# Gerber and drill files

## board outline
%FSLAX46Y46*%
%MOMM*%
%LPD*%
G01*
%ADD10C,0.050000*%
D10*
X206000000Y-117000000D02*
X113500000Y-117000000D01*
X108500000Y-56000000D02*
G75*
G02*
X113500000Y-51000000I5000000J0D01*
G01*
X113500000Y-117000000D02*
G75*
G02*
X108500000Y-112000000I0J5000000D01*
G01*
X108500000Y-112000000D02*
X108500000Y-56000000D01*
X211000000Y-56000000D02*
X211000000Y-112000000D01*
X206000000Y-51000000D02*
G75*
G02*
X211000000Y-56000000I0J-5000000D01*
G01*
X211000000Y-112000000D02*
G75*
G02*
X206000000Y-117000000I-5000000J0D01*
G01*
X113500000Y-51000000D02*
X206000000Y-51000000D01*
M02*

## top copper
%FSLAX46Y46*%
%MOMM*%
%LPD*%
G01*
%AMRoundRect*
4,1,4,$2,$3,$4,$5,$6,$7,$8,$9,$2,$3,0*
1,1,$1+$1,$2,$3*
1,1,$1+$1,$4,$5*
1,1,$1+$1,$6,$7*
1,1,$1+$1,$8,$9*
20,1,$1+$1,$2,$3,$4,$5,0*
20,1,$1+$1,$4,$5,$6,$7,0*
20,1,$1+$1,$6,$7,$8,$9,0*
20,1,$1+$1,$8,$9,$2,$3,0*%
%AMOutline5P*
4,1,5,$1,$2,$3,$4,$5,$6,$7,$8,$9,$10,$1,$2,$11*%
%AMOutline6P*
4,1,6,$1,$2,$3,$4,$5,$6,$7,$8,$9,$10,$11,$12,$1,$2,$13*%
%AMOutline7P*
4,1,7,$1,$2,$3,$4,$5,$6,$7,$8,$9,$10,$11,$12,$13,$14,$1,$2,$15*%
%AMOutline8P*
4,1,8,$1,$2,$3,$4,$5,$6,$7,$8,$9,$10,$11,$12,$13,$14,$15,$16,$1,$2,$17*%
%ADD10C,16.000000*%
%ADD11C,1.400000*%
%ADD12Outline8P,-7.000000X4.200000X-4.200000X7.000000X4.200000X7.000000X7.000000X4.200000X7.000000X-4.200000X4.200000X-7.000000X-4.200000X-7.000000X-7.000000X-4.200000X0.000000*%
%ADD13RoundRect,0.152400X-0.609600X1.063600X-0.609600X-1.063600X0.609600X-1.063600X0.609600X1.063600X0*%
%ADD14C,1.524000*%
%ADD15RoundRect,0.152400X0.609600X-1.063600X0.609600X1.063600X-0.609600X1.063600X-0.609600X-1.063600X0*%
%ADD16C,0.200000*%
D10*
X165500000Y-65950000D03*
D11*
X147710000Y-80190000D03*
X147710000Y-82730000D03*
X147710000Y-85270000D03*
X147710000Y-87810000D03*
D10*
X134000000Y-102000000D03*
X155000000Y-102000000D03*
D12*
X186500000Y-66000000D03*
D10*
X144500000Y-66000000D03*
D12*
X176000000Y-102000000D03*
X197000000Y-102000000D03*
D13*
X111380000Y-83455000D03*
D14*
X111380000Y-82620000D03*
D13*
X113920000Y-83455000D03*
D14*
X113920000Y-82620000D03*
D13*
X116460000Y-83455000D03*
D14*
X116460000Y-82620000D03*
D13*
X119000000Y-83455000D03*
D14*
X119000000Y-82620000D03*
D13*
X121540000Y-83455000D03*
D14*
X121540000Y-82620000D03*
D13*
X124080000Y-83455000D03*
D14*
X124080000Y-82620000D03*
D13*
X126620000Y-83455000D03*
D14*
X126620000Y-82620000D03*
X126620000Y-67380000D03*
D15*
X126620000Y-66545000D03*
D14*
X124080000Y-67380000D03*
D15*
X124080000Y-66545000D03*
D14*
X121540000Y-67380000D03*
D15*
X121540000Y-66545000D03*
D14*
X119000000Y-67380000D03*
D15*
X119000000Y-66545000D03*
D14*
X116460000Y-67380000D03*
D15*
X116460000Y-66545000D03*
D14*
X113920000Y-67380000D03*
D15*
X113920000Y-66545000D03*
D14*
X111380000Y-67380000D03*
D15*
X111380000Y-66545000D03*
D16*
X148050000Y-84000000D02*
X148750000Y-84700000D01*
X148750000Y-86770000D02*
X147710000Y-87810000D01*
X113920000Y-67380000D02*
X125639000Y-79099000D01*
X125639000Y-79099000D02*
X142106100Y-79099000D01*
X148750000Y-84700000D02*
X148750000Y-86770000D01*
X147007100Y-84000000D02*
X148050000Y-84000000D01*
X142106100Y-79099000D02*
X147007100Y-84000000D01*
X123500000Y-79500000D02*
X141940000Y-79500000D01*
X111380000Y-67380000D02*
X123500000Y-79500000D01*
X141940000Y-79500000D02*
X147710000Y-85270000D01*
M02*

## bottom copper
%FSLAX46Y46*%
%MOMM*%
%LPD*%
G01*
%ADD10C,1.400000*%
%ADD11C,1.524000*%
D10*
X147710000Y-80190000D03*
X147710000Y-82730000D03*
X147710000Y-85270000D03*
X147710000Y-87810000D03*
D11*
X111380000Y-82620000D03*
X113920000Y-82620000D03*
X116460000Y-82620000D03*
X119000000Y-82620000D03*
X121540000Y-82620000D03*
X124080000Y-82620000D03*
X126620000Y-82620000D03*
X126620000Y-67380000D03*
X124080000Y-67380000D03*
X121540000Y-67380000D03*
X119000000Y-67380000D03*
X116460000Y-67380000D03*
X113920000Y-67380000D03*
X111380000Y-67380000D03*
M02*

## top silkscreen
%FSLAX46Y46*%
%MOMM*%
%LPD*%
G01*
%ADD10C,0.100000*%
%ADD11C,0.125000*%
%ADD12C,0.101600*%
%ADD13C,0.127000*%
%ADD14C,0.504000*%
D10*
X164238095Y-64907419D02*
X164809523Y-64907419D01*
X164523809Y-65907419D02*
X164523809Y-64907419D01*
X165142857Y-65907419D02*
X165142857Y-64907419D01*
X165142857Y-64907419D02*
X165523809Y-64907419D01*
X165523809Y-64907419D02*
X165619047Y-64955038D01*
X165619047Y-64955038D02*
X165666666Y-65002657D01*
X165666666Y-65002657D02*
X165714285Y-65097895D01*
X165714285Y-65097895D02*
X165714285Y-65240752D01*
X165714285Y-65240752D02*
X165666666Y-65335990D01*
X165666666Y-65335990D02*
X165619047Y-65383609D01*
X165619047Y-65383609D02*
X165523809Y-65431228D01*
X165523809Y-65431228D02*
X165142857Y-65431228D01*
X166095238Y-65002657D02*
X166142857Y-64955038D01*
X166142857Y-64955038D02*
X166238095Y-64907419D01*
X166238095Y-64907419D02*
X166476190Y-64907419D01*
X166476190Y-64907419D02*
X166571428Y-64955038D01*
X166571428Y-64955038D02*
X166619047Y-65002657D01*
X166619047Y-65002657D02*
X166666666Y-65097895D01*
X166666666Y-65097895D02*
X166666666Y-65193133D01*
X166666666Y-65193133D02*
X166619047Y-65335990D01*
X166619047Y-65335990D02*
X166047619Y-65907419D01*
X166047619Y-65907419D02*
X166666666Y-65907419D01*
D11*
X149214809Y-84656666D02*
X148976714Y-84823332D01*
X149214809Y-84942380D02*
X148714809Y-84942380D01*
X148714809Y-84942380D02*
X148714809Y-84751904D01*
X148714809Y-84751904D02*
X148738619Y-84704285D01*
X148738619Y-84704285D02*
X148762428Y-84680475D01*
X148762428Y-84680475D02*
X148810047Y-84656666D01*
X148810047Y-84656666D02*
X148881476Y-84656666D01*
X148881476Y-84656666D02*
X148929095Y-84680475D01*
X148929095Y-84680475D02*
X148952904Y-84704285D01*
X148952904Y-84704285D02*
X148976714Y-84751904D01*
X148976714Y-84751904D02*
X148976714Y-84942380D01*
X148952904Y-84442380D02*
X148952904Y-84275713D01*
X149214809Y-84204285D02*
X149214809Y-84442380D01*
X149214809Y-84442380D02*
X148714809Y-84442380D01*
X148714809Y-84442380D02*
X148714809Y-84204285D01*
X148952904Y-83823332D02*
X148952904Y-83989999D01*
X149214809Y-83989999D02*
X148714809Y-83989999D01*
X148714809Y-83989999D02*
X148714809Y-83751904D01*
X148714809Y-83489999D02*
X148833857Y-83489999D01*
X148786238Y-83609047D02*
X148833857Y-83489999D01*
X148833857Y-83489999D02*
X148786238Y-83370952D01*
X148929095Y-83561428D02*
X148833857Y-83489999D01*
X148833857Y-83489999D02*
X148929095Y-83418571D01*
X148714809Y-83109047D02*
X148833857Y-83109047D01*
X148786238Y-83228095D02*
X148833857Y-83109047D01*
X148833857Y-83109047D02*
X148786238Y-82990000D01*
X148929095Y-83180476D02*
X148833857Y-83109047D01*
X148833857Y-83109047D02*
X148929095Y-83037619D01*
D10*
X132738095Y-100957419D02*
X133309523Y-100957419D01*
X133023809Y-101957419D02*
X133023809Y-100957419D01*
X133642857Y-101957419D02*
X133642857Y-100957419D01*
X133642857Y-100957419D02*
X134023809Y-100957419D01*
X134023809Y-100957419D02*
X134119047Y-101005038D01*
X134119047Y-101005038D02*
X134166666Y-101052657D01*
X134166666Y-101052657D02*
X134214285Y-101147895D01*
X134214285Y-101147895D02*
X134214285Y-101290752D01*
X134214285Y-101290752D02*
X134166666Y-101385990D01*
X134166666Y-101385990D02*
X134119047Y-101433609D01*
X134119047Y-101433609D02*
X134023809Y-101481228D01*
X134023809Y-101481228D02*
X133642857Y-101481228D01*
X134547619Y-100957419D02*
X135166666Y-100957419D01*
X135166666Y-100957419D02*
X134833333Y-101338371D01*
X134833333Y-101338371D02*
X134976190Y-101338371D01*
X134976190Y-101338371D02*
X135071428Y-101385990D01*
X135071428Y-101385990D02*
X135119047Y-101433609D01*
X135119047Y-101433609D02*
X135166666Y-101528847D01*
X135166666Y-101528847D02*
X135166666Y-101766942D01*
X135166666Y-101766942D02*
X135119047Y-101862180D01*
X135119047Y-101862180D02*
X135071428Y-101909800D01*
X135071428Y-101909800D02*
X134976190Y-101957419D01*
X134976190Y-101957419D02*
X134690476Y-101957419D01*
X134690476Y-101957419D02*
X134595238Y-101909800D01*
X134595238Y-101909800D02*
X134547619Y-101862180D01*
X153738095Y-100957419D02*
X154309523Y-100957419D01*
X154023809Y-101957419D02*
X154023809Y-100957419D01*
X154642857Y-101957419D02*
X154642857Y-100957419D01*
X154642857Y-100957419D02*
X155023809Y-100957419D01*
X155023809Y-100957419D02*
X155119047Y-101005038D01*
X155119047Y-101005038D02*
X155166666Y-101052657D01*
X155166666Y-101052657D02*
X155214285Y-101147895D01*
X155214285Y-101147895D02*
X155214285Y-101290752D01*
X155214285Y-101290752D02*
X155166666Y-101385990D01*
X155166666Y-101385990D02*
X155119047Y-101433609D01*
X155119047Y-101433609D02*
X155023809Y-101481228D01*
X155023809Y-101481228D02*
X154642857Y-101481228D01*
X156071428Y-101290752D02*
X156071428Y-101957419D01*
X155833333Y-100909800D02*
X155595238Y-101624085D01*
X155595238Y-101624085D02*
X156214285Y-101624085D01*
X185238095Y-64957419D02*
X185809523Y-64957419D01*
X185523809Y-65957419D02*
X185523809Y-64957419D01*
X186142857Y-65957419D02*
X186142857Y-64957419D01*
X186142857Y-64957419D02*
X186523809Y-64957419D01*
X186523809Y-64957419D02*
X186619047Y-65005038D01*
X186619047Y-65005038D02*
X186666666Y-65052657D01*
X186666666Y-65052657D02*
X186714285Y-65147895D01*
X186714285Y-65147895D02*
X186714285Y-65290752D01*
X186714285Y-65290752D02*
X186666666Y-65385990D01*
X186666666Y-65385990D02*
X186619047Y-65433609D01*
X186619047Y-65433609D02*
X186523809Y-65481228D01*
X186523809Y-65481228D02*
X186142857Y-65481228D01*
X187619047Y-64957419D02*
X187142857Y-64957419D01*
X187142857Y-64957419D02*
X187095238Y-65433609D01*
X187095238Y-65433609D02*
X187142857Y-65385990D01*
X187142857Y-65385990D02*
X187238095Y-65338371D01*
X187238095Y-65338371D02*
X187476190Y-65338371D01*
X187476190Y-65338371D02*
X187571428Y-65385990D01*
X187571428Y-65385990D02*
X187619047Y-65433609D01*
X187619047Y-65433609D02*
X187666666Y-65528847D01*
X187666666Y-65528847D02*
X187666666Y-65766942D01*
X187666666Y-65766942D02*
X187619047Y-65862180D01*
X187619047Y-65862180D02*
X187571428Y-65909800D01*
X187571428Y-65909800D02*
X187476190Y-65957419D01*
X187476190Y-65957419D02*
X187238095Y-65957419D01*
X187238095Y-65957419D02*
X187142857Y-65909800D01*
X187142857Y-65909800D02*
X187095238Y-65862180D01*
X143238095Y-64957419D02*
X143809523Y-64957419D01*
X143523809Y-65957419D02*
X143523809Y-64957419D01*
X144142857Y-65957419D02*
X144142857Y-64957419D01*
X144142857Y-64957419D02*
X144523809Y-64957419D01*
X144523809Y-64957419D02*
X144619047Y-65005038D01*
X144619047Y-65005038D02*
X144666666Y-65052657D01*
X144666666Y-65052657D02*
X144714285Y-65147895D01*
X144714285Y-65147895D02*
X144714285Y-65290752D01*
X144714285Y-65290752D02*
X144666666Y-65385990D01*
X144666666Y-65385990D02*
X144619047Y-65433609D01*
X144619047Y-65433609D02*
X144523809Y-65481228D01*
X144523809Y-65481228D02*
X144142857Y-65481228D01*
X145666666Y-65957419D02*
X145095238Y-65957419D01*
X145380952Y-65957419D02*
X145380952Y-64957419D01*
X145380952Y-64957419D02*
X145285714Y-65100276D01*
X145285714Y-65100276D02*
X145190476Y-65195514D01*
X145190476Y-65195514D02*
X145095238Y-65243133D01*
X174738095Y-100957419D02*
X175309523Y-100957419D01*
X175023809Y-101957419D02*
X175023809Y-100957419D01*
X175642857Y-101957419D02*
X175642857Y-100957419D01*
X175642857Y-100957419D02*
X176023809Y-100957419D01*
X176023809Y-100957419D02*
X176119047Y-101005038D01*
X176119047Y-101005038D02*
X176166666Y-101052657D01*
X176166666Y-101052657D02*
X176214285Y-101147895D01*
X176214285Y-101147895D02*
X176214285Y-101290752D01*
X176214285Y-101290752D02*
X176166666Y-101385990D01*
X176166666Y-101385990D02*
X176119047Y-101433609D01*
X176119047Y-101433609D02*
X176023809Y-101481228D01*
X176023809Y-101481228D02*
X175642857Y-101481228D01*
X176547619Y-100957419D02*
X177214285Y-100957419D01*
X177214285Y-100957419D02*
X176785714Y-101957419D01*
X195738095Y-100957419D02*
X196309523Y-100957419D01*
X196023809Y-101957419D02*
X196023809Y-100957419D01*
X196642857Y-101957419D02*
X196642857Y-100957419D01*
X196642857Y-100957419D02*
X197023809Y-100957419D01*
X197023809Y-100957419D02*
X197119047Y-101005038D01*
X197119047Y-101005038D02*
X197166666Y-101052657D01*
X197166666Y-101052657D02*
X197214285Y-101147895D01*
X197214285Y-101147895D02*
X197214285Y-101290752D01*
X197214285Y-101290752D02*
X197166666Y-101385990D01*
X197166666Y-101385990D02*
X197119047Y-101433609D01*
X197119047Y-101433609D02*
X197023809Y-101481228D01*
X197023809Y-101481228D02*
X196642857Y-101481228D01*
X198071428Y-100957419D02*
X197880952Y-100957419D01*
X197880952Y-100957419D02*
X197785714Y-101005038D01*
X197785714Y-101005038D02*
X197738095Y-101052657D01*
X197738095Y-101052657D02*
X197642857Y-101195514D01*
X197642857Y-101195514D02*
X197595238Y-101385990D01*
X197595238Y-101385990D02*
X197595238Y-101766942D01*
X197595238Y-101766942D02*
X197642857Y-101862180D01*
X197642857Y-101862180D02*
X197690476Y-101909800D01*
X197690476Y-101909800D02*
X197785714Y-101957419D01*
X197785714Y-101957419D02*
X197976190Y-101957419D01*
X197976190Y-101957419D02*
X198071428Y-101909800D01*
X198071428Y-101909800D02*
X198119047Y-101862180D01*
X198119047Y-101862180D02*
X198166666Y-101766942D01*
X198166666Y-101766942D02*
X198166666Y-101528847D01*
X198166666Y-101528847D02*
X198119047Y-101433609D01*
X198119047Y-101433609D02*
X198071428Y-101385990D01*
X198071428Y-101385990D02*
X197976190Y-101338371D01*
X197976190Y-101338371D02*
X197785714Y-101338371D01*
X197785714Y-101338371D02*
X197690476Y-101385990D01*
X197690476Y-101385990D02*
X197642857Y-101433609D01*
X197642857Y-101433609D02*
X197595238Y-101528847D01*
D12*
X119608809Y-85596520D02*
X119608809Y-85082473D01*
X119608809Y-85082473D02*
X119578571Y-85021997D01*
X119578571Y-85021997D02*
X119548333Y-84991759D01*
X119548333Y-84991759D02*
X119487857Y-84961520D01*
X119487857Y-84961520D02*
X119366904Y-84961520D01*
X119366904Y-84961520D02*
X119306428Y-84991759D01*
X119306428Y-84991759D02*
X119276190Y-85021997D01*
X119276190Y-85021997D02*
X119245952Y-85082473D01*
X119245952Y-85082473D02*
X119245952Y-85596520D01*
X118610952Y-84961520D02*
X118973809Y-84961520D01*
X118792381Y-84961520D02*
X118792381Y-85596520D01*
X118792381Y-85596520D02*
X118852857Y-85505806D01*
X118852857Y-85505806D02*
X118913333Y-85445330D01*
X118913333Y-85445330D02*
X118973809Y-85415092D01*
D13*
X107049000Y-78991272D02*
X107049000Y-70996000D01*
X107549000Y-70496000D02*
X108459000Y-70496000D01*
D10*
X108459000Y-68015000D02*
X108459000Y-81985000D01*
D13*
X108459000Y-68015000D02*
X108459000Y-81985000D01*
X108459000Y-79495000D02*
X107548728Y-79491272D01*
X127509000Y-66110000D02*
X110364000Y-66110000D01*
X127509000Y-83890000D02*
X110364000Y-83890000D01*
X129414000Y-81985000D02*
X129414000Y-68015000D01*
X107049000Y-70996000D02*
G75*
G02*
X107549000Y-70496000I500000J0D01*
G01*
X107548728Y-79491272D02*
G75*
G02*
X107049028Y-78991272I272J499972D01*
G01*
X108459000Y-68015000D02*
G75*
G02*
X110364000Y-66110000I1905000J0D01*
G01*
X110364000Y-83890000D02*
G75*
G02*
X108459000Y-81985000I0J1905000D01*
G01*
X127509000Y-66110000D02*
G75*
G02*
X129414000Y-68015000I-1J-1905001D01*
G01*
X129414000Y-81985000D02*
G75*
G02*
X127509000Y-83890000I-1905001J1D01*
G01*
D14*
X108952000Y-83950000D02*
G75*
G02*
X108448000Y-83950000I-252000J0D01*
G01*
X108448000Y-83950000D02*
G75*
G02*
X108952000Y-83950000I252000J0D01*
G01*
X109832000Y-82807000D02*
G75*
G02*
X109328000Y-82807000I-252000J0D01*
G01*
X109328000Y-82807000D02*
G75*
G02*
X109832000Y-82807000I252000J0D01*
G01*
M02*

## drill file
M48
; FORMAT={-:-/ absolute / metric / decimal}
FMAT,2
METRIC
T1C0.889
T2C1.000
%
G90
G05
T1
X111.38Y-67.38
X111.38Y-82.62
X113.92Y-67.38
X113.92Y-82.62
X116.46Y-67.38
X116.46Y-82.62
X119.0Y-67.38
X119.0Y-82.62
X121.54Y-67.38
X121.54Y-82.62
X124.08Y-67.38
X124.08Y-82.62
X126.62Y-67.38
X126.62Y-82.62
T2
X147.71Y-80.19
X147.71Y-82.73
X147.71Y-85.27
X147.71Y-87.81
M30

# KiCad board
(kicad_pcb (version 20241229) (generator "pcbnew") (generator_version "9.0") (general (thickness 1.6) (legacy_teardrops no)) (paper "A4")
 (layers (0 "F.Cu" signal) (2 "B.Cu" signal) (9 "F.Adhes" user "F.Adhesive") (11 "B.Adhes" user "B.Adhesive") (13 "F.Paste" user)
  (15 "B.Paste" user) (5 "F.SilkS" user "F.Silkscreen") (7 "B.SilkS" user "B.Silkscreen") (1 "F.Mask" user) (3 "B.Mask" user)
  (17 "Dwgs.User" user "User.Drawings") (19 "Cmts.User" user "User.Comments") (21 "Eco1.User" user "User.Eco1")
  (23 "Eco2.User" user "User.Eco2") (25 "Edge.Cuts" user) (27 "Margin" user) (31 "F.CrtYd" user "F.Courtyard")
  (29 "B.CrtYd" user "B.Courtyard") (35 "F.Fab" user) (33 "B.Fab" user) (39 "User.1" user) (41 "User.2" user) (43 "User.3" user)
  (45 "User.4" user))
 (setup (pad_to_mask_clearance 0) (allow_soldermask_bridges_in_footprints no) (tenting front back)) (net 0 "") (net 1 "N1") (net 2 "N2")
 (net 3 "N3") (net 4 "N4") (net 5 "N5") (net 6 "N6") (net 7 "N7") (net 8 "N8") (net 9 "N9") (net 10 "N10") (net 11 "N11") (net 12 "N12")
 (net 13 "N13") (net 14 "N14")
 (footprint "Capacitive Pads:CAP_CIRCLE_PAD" (layer "F.Cu") (at 165.5 65.95)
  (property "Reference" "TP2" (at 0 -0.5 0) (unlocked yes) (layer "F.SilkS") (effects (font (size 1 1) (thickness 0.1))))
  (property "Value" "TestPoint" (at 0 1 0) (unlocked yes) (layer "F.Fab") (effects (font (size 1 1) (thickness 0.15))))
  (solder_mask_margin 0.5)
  (pad "1" smd circle (at 0 0) (size 16 16) (layers "F.Cu" "F.Mask" "F.Paste") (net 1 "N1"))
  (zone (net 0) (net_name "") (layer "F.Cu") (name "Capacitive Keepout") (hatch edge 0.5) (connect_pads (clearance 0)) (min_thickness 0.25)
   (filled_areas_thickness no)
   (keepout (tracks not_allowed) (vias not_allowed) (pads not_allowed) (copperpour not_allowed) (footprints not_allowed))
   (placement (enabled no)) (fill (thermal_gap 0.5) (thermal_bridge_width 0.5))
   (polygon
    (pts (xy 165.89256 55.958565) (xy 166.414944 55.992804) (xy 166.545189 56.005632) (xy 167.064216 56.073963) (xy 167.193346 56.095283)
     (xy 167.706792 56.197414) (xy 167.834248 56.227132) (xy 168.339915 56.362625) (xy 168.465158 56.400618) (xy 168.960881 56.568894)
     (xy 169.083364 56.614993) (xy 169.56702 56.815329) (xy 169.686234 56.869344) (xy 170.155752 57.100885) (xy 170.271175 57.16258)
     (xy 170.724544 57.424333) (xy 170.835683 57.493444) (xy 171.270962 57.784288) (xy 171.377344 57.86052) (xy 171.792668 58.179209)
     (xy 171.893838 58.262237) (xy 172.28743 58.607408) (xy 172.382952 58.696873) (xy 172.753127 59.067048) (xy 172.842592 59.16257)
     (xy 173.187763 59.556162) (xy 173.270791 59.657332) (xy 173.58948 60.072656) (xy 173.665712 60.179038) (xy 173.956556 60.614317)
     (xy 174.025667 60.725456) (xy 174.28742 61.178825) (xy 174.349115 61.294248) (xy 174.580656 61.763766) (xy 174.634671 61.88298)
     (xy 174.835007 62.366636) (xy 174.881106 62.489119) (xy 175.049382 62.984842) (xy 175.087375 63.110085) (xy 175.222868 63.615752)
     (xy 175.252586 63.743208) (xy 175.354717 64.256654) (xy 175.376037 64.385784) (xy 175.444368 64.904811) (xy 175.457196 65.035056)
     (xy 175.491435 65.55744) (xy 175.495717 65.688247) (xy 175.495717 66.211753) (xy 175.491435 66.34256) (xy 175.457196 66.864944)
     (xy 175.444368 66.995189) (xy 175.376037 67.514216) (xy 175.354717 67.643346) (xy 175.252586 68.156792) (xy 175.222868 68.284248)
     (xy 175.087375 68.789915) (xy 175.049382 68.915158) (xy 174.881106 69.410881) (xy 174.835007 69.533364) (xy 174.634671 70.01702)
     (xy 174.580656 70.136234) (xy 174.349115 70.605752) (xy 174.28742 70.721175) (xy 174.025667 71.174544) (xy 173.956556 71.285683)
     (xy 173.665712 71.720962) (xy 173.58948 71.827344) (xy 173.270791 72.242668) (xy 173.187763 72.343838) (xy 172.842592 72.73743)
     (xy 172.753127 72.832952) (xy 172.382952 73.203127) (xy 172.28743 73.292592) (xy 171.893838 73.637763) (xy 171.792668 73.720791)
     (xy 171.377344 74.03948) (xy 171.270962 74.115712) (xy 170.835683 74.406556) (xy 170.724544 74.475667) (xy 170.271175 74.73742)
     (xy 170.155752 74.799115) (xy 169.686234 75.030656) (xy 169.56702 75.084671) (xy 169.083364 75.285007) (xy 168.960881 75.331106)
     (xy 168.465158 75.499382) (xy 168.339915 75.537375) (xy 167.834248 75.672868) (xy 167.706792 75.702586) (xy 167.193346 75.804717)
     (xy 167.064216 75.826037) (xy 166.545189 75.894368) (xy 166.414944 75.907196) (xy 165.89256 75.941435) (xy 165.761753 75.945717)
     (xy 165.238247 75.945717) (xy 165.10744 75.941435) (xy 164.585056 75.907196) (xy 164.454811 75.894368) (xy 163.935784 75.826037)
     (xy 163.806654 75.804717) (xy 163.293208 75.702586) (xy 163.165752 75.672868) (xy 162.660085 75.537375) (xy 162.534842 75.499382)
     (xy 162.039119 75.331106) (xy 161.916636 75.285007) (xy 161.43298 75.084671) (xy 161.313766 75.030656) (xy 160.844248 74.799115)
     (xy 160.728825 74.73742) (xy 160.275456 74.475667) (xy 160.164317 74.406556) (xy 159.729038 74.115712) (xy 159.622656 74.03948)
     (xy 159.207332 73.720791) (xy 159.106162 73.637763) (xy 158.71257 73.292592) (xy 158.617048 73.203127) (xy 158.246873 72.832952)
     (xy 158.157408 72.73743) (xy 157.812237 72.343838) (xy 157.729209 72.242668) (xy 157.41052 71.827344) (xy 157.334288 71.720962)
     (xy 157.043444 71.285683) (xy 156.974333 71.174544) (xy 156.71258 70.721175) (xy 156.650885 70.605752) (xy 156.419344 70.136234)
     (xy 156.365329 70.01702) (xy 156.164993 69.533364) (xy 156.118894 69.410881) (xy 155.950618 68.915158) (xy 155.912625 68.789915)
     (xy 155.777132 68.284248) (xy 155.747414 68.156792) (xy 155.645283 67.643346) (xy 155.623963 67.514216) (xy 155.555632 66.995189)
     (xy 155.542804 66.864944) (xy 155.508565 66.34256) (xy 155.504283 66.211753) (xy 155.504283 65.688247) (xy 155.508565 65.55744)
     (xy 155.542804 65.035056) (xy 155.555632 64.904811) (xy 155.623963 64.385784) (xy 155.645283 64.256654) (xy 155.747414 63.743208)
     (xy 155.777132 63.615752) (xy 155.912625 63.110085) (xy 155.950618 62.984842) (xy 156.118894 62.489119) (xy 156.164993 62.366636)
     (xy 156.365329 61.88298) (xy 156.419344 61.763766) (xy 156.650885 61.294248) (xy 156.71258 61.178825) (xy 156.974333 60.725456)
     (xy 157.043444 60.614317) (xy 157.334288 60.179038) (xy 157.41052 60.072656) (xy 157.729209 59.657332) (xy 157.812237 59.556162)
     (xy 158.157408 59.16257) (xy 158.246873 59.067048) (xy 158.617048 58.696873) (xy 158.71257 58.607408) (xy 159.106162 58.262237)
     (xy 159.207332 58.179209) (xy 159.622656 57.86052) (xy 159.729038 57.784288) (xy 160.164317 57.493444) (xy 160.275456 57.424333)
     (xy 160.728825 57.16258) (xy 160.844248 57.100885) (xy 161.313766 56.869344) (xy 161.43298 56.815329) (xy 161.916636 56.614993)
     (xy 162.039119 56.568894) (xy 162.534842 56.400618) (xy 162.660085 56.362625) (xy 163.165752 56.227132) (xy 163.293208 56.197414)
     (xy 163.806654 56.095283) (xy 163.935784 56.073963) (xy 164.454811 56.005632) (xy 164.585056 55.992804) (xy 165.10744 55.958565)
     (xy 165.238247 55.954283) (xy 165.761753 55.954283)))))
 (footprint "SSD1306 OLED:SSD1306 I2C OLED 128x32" (layer "F.Cu") (at 147.71 84 -90)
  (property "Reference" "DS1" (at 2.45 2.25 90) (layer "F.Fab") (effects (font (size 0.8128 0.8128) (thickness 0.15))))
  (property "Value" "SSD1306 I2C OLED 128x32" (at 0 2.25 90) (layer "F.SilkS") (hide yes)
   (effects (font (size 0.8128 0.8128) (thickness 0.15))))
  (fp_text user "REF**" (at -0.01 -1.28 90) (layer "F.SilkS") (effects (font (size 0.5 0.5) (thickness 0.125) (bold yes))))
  (pad "1" thru_hole circle (at -3.81 0 270) (size 1.4 1.4) (drill 1) (layers "*.Cu" "*.Mask") (remove_unused_layers no) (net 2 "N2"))
  (pad "2" thru_hole circle (at -1.27 0 270) (size 1.4 1.4) (drill 1) (layers "*.Cu" "*.Mask") (remove_unused_layers no) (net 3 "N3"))
  (pad "3" thru_hole circle (at 1.27 0 270) (size 1.4 1.4) (drill 1) (layers "*.Cu" "*.Mask") (remove_unused_layers no) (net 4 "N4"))
  (pad "4" thru_hole circle (at 3.81 0 270) (size 1.4 1.4) (drill 1) (layers "*.Cu" "*.Mask") (remove_unused_layers no) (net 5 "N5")))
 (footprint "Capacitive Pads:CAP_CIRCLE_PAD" (layer "F.Cu") (at 134 102)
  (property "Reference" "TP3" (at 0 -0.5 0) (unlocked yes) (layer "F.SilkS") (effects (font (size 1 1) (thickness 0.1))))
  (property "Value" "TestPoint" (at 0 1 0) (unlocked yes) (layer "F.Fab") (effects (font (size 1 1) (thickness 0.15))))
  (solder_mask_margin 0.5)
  (pad "1" smd circle (at 0 0) (size 16 16) (layers "F.Cu" "F.Mask" "F.Paste") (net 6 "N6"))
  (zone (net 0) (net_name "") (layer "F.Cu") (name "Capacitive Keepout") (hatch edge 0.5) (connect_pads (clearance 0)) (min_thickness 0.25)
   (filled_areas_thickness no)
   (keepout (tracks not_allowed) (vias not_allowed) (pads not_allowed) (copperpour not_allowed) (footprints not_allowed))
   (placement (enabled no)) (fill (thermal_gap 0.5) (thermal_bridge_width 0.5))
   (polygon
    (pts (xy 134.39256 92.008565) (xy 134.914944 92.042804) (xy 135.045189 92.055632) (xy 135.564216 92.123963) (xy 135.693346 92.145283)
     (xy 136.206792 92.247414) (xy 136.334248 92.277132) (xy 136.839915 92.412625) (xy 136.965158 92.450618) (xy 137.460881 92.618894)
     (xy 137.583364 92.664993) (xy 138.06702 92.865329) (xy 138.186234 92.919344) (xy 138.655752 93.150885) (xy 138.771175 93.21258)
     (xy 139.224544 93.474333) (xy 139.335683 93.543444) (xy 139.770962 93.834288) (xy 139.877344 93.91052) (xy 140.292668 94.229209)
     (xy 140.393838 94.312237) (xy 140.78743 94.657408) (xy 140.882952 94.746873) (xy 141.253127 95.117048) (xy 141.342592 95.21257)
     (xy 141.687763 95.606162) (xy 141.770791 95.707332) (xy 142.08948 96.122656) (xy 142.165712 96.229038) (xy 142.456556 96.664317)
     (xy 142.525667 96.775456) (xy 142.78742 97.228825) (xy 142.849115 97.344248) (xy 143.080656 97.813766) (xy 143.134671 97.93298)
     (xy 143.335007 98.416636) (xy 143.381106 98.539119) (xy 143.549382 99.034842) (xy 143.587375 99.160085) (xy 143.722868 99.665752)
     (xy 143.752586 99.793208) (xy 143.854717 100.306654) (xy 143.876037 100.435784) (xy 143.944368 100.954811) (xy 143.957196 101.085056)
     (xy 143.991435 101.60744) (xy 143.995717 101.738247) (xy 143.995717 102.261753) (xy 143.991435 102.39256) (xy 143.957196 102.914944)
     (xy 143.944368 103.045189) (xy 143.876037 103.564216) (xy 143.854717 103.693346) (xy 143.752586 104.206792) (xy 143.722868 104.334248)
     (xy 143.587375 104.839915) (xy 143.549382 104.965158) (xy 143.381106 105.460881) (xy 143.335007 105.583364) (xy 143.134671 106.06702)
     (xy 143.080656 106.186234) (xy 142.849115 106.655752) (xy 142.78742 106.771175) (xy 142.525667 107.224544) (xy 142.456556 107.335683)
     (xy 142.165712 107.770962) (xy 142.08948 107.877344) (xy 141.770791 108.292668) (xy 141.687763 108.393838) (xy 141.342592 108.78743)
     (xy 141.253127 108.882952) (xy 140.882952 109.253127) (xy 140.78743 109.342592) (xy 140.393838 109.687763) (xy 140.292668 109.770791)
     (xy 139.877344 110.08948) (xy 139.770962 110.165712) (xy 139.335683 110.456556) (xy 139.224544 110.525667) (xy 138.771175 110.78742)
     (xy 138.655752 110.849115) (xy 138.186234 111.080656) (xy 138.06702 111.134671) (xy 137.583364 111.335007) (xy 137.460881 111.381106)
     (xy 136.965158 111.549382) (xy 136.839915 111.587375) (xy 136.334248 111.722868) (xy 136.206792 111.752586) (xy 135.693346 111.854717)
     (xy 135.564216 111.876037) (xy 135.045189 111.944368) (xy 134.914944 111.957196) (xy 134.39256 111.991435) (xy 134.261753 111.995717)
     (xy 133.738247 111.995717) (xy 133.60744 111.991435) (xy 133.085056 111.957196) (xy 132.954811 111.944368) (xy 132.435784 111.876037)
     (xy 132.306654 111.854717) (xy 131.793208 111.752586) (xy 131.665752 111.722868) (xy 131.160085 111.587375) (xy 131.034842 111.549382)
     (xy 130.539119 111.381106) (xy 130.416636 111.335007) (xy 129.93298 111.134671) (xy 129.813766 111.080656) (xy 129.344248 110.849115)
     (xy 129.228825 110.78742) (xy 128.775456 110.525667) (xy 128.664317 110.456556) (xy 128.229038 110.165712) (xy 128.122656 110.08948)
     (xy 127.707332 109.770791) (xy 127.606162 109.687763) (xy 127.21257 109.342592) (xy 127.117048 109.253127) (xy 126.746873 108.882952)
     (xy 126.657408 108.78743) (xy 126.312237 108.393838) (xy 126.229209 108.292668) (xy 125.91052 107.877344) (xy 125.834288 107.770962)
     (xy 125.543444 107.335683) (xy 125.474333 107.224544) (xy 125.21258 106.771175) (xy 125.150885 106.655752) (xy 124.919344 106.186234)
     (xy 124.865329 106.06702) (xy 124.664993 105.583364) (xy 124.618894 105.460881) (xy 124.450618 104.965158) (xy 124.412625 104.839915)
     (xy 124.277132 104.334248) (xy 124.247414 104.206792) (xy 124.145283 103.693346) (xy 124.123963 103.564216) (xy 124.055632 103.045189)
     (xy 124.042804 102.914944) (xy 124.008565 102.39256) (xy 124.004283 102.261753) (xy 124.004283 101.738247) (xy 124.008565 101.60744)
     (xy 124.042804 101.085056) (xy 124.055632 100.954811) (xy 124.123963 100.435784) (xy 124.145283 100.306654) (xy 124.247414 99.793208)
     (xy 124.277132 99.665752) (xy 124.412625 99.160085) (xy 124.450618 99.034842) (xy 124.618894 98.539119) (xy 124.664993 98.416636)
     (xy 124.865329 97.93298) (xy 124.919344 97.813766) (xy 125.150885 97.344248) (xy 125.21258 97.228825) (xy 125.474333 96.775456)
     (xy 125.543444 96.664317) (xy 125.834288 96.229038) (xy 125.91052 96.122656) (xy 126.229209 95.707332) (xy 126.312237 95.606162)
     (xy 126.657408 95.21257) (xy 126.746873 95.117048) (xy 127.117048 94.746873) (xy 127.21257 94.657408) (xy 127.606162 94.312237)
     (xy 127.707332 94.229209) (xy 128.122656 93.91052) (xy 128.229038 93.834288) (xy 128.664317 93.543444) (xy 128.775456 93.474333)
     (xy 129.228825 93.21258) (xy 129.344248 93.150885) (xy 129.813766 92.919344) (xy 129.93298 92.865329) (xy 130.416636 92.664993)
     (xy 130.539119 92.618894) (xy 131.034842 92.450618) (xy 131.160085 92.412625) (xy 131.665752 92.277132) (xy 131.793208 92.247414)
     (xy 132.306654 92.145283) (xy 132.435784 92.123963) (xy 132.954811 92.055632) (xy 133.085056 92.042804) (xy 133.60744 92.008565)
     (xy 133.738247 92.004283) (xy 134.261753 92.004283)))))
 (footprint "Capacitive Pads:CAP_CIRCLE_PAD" (layer "F.Cu") (at 155 102)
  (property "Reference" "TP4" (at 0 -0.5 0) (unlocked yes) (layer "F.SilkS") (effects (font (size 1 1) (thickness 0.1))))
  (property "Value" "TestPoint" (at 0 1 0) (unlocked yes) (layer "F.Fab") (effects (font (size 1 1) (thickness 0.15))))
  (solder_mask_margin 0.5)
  (pad "1" smd circle (at 0 0) (size 16 16) (layers "F.Cu" "F.Mask" "F.Paste") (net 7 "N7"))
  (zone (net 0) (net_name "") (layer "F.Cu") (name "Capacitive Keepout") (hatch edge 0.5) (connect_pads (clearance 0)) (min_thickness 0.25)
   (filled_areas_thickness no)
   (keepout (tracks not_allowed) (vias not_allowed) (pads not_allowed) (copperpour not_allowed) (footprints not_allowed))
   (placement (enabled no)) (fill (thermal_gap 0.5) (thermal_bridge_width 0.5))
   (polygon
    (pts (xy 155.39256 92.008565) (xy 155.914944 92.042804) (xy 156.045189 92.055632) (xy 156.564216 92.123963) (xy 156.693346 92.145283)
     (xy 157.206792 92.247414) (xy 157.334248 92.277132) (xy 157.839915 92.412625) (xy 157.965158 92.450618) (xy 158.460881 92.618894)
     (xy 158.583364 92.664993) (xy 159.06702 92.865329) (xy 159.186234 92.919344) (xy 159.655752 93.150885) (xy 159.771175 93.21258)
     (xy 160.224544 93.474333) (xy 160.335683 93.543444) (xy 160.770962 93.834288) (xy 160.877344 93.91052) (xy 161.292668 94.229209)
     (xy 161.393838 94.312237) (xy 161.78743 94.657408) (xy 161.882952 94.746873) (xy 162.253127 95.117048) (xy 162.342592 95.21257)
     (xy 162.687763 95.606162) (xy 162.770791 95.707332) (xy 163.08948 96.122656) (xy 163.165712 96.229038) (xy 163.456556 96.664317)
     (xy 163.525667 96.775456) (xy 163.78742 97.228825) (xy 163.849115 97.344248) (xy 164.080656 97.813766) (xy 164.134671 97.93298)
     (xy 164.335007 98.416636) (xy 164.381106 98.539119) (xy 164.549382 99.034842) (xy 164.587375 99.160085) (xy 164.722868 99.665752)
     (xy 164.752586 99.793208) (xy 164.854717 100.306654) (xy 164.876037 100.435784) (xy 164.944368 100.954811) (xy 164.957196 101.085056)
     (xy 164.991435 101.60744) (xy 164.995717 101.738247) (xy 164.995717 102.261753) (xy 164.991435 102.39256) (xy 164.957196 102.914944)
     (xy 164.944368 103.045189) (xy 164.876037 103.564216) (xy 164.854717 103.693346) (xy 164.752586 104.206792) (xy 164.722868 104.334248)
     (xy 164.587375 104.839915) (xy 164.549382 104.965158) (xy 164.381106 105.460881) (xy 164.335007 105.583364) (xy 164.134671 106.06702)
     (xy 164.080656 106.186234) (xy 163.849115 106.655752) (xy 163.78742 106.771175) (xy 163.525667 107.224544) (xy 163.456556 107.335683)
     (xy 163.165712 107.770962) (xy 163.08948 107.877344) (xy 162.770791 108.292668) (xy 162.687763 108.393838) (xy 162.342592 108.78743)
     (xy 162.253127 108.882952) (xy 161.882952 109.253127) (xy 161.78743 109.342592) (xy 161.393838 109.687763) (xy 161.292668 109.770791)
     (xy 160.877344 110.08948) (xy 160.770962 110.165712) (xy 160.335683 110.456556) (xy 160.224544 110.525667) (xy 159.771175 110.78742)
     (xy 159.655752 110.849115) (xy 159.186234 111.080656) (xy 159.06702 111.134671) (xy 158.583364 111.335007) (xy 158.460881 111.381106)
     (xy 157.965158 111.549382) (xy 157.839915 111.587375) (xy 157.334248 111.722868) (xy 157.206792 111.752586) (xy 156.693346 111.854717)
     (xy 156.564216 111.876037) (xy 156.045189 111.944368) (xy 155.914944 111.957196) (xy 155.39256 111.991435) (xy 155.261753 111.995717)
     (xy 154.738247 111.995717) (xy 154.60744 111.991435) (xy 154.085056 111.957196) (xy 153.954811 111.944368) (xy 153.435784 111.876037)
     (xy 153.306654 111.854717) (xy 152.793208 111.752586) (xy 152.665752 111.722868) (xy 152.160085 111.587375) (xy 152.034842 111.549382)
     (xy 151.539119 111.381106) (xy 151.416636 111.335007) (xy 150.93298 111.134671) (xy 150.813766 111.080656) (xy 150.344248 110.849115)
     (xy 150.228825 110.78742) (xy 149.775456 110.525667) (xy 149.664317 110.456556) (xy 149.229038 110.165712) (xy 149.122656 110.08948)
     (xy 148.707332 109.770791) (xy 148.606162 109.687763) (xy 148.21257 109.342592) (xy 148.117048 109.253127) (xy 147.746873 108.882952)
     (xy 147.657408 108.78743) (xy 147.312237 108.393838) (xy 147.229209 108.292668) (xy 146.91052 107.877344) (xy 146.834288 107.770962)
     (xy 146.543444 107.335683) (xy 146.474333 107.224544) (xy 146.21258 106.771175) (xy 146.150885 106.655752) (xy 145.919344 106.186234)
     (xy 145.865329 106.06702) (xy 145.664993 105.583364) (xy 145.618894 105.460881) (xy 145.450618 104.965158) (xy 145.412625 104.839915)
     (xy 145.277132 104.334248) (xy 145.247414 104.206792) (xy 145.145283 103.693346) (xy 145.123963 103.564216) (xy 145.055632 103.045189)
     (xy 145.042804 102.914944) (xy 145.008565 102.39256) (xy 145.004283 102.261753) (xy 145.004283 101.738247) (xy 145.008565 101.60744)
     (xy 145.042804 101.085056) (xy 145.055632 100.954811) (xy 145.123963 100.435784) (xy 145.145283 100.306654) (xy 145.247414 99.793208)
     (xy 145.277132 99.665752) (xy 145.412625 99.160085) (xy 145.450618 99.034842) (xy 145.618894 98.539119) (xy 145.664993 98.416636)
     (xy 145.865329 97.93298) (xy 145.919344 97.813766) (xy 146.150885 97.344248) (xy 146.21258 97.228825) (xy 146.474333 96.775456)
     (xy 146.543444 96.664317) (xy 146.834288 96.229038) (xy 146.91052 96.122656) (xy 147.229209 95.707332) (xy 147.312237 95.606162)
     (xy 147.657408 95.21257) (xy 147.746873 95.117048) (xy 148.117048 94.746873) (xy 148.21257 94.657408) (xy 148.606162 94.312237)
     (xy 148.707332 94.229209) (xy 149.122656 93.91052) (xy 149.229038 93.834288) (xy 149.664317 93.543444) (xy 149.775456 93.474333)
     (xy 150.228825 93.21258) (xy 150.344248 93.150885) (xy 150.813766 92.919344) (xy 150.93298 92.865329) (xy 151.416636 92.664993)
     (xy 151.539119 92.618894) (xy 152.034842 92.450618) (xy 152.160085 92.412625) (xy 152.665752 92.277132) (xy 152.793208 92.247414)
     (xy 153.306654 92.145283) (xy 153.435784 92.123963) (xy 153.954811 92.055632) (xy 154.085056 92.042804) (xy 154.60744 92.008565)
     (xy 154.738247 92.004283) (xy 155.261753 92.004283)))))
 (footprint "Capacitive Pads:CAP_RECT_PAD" (layer "F.Cu") (at 186.5 66)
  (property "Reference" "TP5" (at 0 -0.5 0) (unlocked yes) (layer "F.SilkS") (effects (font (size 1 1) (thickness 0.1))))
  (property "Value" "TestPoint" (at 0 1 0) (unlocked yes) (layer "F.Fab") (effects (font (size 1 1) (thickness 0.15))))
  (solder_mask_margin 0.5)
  (pad "1" smd roundrect (at 0 0) (size 14 14) (layers "F.Cu" "F.Mask" "F.Paste") (roundrect_rratio 0) (chamfer_ratio 0.2)
   (chamfer top_left top_right bottom_left bottom_right) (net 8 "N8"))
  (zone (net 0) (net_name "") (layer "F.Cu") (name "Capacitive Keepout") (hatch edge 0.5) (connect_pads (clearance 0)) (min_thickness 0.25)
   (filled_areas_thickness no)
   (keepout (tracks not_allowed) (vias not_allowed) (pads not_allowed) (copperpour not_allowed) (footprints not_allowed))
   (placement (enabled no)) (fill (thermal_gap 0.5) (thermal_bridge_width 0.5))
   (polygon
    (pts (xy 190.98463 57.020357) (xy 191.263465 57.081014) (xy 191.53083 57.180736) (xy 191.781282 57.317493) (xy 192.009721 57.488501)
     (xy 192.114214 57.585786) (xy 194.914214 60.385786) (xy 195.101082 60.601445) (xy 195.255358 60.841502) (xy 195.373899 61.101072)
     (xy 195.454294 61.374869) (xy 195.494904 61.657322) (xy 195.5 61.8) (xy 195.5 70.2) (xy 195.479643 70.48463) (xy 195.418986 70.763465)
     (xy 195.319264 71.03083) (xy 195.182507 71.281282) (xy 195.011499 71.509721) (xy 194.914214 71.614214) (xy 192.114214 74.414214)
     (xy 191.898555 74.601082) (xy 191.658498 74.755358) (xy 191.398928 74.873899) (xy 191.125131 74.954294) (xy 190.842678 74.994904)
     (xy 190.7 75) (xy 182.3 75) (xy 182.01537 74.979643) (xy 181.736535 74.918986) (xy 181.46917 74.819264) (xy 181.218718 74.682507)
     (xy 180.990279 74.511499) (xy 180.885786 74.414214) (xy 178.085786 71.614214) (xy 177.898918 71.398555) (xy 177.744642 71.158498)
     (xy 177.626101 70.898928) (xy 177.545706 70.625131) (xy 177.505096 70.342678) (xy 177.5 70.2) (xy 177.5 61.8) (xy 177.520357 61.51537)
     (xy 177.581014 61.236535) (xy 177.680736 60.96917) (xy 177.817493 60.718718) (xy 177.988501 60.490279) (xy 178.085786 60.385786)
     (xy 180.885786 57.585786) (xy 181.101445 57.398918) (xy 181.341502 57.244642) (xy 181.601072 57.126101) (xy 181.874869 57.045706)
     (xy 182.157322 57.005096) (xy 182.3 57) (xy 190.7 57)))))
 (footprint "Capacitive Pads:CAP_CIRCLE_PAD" (layer "F.Cu") (at 144.5 66)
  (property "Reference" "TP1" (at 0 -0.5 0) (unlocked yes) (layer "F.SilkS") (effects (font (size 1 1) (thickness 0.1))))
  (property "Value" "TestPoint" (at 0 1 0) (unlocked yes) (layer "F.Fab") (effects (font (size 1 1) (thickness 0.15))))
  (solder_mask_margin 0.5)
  (pad "1" smd circle (at 0 0) (size 16 16) (layers "F.Cu" "F.Mask" "F.Paste") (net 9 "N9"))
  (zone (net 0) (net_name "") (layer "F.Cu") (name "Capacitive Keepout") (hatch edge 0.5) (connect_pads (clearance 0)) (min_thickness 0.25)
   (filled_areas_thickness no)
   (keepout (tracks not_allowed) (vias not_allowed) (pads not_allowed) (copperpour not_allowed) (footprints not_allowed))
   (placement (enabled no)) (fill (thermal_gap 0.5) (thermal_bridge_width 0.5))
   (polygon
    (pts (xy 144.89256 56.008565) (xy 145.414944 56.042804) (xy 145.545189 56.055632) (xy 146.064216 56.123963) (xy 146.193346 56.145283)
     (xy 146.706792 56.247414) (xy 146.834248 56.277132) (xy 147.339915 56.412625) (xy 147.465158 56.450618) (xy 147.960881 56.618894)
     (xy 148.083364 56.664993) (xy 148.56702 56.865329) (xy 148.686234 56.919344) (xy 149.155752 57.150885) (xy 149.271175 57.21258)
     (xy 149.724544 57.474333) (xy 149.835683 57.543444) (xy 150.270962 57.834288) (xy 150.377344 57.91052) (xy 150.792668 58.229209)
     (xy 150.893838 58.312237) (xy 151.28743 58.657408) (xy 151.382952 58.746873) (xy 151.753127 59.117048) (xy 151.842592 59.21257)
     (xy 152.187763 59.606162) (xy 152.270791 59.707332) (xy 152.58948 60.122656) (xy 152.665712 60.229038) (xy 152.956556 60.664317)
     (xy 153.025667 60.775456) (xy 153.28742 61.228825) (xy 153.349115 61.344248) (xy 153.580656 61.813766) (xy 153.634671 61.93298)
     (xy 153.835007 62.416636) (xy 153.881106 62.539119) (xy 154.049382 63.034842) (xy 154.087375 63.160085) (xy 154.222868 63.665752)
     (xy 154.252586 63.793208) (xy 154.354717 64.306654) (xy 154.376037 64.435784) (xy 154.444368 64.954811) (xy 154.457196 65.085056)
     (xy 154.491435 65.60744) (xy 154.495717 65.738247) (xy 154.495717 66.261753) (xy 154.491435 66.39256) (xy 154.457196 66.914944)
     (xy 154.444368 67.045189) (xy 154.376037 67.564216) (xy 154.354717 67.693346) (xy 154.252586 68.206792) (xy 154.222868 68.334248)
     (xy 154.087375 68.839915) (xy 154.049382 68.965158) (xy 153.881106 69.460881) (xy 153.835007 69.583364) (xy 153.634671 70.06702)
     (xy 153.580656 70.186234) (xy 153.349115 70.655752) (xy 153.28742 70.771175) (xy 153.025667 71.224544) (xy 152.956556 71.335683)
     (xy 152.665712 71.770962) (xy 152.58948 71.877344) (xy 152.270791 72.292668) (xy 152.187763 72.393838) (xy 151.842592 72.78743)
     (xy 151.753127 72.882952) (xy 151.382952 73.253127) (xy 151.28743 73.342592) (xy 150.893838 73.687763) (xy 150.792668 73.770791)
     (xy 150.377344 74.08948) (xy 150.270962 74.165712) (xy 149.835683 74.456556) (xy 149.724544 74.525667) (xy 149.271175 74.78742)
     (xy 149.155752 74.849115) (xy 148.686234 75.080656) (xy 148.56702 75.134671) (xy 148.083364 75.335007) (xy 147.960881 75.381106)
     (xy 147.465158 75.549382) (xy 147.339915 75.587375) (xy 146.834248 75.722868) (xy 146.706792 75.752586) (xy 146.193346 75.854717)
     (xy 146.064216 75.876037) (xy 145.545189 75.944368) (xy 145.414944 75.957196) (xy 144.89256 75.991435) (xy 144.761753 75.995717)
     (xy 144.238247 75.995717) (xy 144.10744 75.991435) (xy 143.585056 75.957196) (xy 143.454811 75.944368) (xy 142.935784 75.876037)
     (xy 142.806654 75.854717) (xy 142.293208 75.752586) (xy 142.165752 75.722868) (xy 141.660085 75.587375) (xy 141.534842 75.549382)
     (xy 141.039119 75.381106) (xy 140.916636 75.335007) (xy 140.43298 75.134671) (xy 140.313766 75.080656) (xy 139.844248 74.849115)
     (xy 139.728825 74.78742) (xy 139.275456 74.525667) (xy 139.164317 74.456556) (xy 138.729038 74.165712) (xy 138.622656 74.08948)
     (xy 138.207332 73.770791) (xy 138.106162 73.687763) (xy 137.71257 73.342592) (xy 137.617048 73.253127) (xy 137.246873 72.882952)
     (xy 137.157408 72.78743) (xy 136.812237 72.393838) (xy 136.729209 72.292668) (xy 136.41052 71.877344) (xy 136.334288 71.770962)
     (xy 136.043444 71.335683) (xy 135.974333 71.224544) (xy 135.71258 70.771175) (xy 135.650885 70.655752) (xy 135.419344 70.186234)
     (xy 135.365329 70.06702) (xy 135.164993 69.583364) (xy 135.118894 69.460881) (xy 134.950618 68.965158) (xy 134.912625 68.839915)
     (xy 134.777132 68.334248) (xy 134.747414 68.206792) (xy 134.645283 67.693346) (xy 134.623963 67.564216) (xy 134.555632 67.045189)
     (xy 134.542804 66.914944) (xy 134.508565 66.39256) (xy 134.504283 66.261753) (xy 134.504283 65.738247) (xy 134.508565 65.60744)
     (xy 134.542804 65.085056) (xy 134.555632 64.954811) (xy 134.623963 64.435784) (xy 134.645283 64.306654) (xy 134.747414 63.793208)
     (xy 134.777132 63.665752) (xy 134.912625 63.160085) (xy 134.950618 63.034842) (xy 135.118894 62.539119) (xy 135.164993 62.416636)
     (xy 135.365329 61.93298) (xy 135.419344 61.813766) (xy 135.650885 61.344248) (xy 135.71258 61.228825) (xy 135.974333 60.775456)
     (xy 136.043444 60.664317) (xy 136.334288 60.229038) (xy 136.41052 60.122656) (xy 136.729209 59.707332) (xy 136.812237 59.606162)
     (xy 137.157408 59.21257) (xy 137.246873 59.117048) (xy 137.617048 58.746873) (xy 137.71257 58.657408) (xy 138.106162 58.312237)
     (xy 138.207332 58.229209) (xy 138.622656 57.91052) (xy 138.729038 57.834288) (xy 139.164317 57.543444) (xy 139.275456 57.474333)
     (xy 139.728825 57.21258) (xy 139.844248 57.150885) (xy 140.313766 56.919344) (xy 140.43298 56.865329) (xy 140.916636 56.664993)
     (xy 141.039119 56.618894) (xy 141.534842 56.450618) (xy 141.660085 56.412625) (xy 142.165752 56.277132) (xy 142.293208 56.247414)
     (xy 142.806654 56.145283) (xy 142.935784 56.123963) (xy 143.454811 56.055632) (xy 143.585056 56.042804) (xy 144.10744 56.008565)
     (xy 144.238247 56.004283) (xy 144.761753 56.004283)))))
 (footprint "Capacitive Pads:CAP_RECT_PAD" (layer "F.Cu") (at 176 102)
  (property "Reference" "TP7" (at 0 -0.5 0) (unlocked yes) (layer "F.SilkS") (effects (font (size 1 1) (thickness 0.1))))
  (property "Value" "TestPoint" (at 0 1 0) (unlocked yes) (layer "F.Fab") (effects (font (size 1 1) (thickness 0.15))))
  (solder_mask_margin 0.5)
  (pad "1" smd roundrect (at 0 0) (size 14 14) (layers "F.Cu" "F.Mask" "F.Paste") (roundrect_rratio 0) (chamfer_ratio 0.2)
   (chamfer top_left top_right bottom_left bottom_right) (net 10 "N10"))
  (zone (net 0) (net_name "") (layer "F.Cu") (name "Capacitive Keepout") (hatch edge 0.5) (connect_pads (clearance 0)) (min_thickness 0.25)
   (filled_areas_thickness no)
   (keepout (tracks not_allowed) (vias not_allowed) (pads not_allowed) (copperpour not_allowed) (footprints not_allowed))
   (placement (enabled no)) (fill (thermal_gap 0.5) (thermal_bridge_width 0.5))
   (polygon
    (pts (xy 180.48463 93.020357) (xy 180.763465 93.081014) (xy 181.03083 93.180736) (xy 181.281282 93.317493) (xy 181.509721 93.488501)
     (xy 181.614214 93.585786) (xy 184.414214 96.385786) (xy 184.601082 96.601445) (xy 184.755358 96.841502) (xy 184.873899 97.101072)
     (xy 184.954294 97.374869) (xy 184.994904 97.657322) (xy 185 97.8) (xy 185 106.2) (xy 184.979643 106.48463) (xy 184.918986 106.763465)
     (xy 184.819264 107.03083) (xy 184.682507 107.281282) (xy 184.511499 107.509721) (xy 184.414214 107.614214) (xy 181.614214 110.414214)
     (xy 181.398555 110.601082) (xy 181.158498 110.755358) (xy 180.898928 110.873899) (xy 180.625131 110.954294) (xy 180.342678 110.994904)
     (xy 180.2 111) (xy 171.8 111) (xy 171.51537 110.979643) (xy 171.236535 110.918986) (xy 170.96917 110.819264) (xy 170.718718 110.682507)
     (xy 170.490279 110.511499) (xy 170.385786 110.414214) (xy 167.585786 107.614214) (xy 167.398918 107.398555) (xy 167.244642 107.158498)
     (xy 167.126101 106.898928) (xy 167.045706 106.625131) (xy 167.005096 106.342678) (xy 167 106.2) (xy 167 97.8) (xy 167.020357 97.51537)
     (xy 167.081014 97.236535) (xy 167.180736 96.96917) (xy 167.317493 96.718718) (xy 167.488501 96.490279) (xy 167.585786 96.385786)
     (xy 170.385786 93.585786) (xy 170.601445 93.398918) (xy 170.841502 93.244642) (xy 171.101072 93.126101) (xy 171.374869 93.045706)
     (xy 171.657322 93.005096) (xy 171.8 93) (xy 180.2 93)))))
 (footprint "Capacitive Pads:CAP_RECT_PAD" (layer "F.Cu") (at 197 102)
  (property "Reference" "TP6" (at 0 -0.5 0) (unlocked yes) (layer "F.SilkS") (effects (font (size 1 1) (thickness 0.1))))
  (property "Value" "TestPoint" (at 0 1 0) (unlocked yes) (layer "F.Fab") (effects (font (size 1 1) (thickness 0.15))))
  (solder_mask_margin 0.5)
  (pad "1" smd roundrect (at 0 0) (size 14 14) (layers "F.Cu" "F.Mask" "F.Paste") (roundrect_rratio 0) (chamfer_ratio 0.2)
   (chamfer top_left top_right bottom_left bottom_right) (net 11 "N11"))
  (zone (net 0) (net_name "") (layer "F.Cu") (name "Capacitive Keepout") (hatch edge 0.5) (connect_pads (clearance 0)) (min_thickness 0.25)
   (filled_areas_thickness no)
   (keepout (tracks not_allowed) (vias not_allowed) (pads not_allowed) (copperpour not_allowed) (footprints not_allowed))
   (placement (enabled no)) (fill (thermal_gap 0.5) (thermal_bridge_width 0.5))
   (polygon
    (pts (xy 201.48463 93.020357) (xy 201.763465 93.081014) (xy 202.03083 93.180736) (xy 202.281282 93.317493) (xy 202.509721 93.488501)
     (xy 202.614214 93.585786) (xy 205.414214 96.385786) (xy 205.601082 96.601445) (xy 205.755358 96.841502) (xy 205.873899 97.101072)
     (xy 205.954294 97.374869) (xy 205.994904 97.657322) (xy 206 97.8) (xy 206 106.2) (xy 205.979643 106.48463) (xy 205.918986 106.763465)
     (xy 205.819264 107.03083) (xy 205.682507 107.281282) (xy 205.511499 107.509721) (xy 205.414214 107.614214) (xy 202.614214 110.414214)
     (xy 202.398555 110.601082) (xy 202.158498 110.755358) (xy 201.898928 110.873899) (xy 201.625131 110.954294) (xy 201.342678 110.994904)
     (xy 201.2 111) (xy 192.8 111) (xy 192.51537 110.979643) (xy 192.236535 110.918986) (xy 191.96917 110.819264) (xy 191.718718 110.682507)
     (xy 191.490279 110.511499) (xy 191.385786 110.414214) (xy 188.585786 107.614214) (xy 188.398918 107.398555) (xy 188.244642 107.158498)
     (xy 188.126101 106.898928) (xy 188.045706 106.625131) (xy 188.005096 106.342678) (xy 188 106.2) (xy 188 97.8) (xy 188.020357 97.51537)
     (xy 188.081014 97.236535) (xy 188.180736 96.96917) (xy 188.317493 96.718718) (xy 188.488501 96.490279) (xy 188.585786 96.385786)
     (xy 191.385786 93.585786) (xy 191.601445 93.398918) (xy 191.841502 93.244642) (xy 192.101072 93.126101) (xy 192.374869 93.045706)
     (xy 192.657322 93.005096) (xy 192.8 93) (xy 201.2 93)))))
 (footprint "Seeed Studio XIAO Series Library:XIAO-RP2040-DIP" (layer "F.Cu") (at 119 75 180)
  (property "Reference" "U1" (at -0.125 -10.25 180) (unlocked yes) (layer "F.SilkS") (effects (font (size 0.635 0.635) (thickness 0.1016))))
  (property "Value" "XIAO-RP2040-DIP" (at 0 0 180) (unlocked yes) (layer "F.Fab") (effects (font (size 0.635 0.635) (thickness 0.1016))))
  (fp_line (start 11.951 -3.991272) (end 11.951 4.004) (stroke (width 0.127) (type solid)) (layer "F.SilkS"))
  (fp_line (start 11.451 4.504) (end 10.541 4.504) (stroke (width 0.127) (type solid)) (layer "F.SilkS"))
  (fp_line (start 10.541 6.985) (end 10.541 -6.985) (stroke (width 0.1) (type solid)) (layer "F.SilkS"))
  (fp_line (start 10.541 6.985) (end 10.541 -6.985) (stroke (width 0.127) (type solid)) (layer "F.SilkS"))
  (fp_line (start 10.541 -4.495) (end 11.451272 -4.491272) (stroke (width 0.127) (type solid)) (layer "F.SilkS"))
  (fp_line (start -8.509 8.89) (end 8.636 8.89) (stroke (width 0.127) (type solid)) (layer "F.SilkS"))
  (fp_line (start -8.509 -8.89) (end 8.636 -8.89) (stroke (width 0.127) (type solid)) (layer "F.SilkS"))
  (fp_line (start -10.414 -6.985) (end -10.414 6.985) (stroke (width 0.127) (type solid)) (layer "F.SilkS"))
  (fp_arc (start 11.951 4.004) (mid 11.804553 4.357553) (end 11.451 4.504) (stroke (width 0.127) (type default)) (layer "F.SilkS"))
  (fp_arc (start 11.451272 -4.491272) (mid 11.804644 -4.344724) (end 11.951 -3.991272) (stroke (width 0.127) (type default))
   (layer "F.SilkS"))
  (fp_arc (start 10.541 6.985) (mid 9.983038 8.332038) (end 8.636 8.89) (stroke (width 0.127) (type solid)) (layer "F.SilkS"))
  (fp_arc (start 8.636 -8.89) (mid 9.983038 -8.332038) (end 10.541 -6.985) (stroke (width 0.127) (type solid)) (layer "F.SilkS"))
  (fp_arc (start -8.509 8.89) (mid -9.856038 8.332038) (end -10.414 6.985) (stroke (width 0.127) (type solid)) (layer "F.SilkS"))
  (fp_arc (start -10.414 -6.985) (mid -9.856038 -8.332038) (end -8.509 -8.89) (stroke (width 0.127) (type solid)) (layer "F.SilkS"))
  (fp_circle (center 10.3 -8.95) (end 10.554 -8.95) (stroke (width 0.5) (type solid)) (fill yes) (layer "F.SilkS"))
  (fp_circle (center 9.42 -7.807) (end 9.674 -7.807) (stroke (width 0.5) (type solid)) (fill yes) (layer "F.SilkS"))
  (pad "1" smd roundrect (at 7.62 -8.455 270) (size 2.432 1.524) (layers "F.Cu" "F.Mask") (roundrect_rratio 0.1) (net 9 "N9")
   (thermal_bridge_angle 45))
  (pad "1" thru_hole circle (at 7.62 -7.62 270) (size 1.524 1.524) (drill 0.889) (layers "*.Cu" "*.Mask") (remove_unused_layers no)
   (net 9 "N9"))
  (pad "2" smd roundrect (at 5.08 -8.455 270) (size 2.432 1.524) (layers "F.Cu" "F.Mask") (roundrect_rratio 0.1) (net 1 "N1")
   (thermal_bridge_angle 45))
  (pad "2" thru_hole circle (at 5.08 -7.62 270) (size 1.524 1.524) (drill 0.889) (layers "*.Cu" "*.Mask") (remove_unused_layers no)
   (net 1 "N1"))
  (pad "3" smd roundrect (at 2.54 -8.455 270) (size 2.432 1.524) (layers "F.Cu" "F.Mask") (roundrect_rratio 0.1) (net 6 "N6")
   (thermal_bridge_angle 45))
  (pad "3" thru_hole circle (at 2.54 -7.62 270) (size 1.524 1.524) (drill 0.889) (layers "*.Cu" "*.Mask") (remove_unused_layers no)
   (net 6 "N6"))
  (pad "4" smd roundrect (at 0 -8.455 270) (size 2.432 1.524) (layers "F.Cu" "F.Mask") (roundrect_rratio 0.1) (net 7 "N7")
   (thermal_bridge_angle 45))
  (pad "4" thru_hole circle (at 0 -7.62 270) (size 1.524 1.524) (drill 0.889) (layers "*.Cu" "*.Mask") (remove_unused_layers no)
   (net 7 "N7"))
  (pad "5" smd roundrect (at -2.54 -8.455 270) (size 2.432 1.524) (layers "F.Cu" "F.Mask") (roundrect_rratio 0.1) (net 2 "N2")
   (thermal_bridge_angle 45))
  (pad "5" thru_hole circle (at -2.54 -7.62 270) (size 1.524 1.524) (drill 0.889) (layers "*.Cu" "*.Mask") (remove_unused_layers no)
   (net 2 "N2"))
  (pad "6" smd roundrect (at -5.08 -8.455 270) (size 2.432 1.524) (layers "F.Cu" "F.Mask") (roundrect_rratio 0.1) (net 3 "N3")
   (thermal_bridge_angle 45))
  (pad "6" thru_hole circle (at -5.08 -7.62 270) (size 1.524 1.524) (drill 0.889) (layers "*.Cu" "*.Mask") (remove_unused_layers no)
   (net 3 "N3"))
  (pad "7" smd roundrect (at -7.62 -8.455 270) (size 2.432 1.524) (layers "F.Cu" "F.Mask") (roundrect_rratio 0.1) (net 8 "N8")
   (thermal_bridge_angle 45))
  (pad "7" thru_hole circle (at -7.62 -7.62 270) (size 1.524 1.524) (drill 0.889) (layers "*.Cu" "*.Mask") (remove_unused_layers no)
   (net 8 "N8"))
  (pad "8" thru_hole circle (at -7.62 7.62 90) (size 1.524 1.524) (drill 0.889) (layers "*.Cu" "*.Mask") (remove_unused_layers no)
   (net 10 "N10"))
  (pad "8" smd roundrect (at -7.62 8.455 90) (size 2.432 1.524) (layers "F.Cu" "F.Mask") (roundrect_rratio 0.1) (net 10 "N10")
   (thermal_bridge_angle 45))
  (pad "9" thru_hole circle (at -5.08 7.62 90) (size 1.524 1.524) (drill 0.889) (layers "*.Cu" "*.Mask") (remove_unused_layers no)
   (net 11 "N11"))
  (pad "9" smd roundrect (at -5.08 8.455 90) (size 2.432 1.524) (layers "F.Cu" "F.Mask") (roundrect_rratio 0.1) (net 11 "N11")
   (thermal_bridge_angle 45))
  (pad "10" thru_hole circle (at -2.54 7.62 90) (size 1.524 1.524) (drill 0.889) (layers "*.Cu" "*.Mask") (remove_unused_layers no)
   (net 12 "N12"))
  (pad "10" smd roundrect (at -2.54 8.455 90) (size 2.432 1.524) (layers "F.Cu" "F.Mask") (roundrect_rratio 0.1) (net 12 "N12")
   (thermal_bridge_angle 45))
  (pad "11" thru_hole circle (at 0 7.62 90) (size 1.524 1.524) (drill 0.889) (layers "*.Cu" "*.Mask") (remove_unused_layers no)
   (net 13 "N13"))
  (pad "11" smd roundrect (at 0 8.455 90) (size 2.432 1.524) (layers "F.Cu" "F.Mask") (roundrect_rratio 0.1) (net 13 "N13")
   (thermal_bridge_angle 45))
  (pad "12" thru_hole circle (at 2.54 7.62 90) (size 1.524 1.524) (drill 0.889) (layers "*.Cu" "*.Mask") (remove_unused_layers no)
   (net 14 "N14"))
  (pad "12" smd roundrect (at 2.54 8.455 90) (size 2.432 1.524) (layers "F.Cu" "F.Mask") (roundrect_rratio 0.1) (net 14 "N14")
   (thermal_bridge_angle 45))
  (pad "13" thru_hole circle (at 5.08 7.62 90) (size 1.524 1.524) (drill 0.889) (layers "*.Cu" "*.Mask") (remove_unused_layers no)
   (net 5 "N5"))
  (pad "13" smd roundrect (at 5.08 8.455 90) (size 2.432 1.524) (layers "F.Cu" "F.Mask") (roundrect_rratio 0.1) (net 5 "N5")
   (thermal_bridge_angle 45))
  (pad "14" thru_hole circle (at 7.62 7.62 90) (size 1.524 1.524) (drill 0.889) (layers "*.Cu" "*.Mask") (remove_unused_layers no)
   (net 4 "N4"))
  (pad "14" smd roundrect (at 7.62 8.455 90) (size 2.432 1.524) (layers "F.Cu" "F.Mask") (roundrect_rratio 0.1) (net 4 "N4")
   (thermal_bridge_angle 45)))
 (gr_line (start 206 117) (end 113.5 117) (stroke (width 0.05) (type default)) (layer "Edge.Cuts"))
 (gr_arc (start 108.5 56) (mid 109.964466 52.464466) (end 113.5 51) (stroke (width 0.05) (type default)) (layer "Edge.Cuts"))
 (gr_arc (start 113.5 117) (mid 109.964466 115.535534) (end 108.5 112) (stroke (width 0.05) (type default)) (layer "Edge.Cuts"))
 (gr_line (start 108.5 112) (end 108.5 56) (stroke (width 0.05) (type default)) (layer "Edge.Cuts"))
 (gr_line (start 211 56) (end 211 112) (stroke (width 0.05) (type default)) (layer "Edge.Cuts"))
 (gr_arc (start 206 51) (mid 209.535534 52.464466) (end 211 56) (stroke (width 0.05) (type default)) (layer "Edge.Cuts"))
 (gr_arc (start 211 112) (mid 209.535534 115.535534) (end 206 117) (stroke (width 0.05) (type default)) (layer "Edge.Cuts"))
 (gr_line (start 113.5 51) (end 206 51) (stroke (width 0.05) (type default)) (layer "Edge.Cuts"))
 (segment (start 148.05 84) (end 148.75 84.7) (width 0.2) (layer "F.Cu") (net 5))
 (segment (start 148.75 86.77) (end 147.71 87.81) (width 0.2) (layer "F.Cu") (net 5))
 (segment (start 113.92 67.38) (end 125.639 79.099) (width 0.2) (layer "F.Cu") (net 5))
 (segment (start 125.639 79.099) (end 142.1061 79.099) (width 0.2) (layer "F.Cu") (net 5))
 (segment (start 148.75 84.7) (end 148.75 86.77) (width 0.2) (layer "F.Cu") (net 5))
 (segment (start 147.0071 84) (end 148.05 84) (width 0.2) (layer "F.Cu") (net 5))
 (segment (start 142.1061 79.099) (end 147.0071 84) (width 0.2) (layer "F.Cu") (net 5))
 (segment (start 123.5 79.5) (end 141.94 79.5) (width 0.2) (layer "F.Cu") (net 4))
 (segment (start 111.38 67.38) (end 123.5 79.5) (width 0.2) (layer "F.Cu") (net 4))
 (segment (start 141.94 79.5) (end 147.71 85.27) (width 0.2) (layer "F.Cu") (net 4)))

